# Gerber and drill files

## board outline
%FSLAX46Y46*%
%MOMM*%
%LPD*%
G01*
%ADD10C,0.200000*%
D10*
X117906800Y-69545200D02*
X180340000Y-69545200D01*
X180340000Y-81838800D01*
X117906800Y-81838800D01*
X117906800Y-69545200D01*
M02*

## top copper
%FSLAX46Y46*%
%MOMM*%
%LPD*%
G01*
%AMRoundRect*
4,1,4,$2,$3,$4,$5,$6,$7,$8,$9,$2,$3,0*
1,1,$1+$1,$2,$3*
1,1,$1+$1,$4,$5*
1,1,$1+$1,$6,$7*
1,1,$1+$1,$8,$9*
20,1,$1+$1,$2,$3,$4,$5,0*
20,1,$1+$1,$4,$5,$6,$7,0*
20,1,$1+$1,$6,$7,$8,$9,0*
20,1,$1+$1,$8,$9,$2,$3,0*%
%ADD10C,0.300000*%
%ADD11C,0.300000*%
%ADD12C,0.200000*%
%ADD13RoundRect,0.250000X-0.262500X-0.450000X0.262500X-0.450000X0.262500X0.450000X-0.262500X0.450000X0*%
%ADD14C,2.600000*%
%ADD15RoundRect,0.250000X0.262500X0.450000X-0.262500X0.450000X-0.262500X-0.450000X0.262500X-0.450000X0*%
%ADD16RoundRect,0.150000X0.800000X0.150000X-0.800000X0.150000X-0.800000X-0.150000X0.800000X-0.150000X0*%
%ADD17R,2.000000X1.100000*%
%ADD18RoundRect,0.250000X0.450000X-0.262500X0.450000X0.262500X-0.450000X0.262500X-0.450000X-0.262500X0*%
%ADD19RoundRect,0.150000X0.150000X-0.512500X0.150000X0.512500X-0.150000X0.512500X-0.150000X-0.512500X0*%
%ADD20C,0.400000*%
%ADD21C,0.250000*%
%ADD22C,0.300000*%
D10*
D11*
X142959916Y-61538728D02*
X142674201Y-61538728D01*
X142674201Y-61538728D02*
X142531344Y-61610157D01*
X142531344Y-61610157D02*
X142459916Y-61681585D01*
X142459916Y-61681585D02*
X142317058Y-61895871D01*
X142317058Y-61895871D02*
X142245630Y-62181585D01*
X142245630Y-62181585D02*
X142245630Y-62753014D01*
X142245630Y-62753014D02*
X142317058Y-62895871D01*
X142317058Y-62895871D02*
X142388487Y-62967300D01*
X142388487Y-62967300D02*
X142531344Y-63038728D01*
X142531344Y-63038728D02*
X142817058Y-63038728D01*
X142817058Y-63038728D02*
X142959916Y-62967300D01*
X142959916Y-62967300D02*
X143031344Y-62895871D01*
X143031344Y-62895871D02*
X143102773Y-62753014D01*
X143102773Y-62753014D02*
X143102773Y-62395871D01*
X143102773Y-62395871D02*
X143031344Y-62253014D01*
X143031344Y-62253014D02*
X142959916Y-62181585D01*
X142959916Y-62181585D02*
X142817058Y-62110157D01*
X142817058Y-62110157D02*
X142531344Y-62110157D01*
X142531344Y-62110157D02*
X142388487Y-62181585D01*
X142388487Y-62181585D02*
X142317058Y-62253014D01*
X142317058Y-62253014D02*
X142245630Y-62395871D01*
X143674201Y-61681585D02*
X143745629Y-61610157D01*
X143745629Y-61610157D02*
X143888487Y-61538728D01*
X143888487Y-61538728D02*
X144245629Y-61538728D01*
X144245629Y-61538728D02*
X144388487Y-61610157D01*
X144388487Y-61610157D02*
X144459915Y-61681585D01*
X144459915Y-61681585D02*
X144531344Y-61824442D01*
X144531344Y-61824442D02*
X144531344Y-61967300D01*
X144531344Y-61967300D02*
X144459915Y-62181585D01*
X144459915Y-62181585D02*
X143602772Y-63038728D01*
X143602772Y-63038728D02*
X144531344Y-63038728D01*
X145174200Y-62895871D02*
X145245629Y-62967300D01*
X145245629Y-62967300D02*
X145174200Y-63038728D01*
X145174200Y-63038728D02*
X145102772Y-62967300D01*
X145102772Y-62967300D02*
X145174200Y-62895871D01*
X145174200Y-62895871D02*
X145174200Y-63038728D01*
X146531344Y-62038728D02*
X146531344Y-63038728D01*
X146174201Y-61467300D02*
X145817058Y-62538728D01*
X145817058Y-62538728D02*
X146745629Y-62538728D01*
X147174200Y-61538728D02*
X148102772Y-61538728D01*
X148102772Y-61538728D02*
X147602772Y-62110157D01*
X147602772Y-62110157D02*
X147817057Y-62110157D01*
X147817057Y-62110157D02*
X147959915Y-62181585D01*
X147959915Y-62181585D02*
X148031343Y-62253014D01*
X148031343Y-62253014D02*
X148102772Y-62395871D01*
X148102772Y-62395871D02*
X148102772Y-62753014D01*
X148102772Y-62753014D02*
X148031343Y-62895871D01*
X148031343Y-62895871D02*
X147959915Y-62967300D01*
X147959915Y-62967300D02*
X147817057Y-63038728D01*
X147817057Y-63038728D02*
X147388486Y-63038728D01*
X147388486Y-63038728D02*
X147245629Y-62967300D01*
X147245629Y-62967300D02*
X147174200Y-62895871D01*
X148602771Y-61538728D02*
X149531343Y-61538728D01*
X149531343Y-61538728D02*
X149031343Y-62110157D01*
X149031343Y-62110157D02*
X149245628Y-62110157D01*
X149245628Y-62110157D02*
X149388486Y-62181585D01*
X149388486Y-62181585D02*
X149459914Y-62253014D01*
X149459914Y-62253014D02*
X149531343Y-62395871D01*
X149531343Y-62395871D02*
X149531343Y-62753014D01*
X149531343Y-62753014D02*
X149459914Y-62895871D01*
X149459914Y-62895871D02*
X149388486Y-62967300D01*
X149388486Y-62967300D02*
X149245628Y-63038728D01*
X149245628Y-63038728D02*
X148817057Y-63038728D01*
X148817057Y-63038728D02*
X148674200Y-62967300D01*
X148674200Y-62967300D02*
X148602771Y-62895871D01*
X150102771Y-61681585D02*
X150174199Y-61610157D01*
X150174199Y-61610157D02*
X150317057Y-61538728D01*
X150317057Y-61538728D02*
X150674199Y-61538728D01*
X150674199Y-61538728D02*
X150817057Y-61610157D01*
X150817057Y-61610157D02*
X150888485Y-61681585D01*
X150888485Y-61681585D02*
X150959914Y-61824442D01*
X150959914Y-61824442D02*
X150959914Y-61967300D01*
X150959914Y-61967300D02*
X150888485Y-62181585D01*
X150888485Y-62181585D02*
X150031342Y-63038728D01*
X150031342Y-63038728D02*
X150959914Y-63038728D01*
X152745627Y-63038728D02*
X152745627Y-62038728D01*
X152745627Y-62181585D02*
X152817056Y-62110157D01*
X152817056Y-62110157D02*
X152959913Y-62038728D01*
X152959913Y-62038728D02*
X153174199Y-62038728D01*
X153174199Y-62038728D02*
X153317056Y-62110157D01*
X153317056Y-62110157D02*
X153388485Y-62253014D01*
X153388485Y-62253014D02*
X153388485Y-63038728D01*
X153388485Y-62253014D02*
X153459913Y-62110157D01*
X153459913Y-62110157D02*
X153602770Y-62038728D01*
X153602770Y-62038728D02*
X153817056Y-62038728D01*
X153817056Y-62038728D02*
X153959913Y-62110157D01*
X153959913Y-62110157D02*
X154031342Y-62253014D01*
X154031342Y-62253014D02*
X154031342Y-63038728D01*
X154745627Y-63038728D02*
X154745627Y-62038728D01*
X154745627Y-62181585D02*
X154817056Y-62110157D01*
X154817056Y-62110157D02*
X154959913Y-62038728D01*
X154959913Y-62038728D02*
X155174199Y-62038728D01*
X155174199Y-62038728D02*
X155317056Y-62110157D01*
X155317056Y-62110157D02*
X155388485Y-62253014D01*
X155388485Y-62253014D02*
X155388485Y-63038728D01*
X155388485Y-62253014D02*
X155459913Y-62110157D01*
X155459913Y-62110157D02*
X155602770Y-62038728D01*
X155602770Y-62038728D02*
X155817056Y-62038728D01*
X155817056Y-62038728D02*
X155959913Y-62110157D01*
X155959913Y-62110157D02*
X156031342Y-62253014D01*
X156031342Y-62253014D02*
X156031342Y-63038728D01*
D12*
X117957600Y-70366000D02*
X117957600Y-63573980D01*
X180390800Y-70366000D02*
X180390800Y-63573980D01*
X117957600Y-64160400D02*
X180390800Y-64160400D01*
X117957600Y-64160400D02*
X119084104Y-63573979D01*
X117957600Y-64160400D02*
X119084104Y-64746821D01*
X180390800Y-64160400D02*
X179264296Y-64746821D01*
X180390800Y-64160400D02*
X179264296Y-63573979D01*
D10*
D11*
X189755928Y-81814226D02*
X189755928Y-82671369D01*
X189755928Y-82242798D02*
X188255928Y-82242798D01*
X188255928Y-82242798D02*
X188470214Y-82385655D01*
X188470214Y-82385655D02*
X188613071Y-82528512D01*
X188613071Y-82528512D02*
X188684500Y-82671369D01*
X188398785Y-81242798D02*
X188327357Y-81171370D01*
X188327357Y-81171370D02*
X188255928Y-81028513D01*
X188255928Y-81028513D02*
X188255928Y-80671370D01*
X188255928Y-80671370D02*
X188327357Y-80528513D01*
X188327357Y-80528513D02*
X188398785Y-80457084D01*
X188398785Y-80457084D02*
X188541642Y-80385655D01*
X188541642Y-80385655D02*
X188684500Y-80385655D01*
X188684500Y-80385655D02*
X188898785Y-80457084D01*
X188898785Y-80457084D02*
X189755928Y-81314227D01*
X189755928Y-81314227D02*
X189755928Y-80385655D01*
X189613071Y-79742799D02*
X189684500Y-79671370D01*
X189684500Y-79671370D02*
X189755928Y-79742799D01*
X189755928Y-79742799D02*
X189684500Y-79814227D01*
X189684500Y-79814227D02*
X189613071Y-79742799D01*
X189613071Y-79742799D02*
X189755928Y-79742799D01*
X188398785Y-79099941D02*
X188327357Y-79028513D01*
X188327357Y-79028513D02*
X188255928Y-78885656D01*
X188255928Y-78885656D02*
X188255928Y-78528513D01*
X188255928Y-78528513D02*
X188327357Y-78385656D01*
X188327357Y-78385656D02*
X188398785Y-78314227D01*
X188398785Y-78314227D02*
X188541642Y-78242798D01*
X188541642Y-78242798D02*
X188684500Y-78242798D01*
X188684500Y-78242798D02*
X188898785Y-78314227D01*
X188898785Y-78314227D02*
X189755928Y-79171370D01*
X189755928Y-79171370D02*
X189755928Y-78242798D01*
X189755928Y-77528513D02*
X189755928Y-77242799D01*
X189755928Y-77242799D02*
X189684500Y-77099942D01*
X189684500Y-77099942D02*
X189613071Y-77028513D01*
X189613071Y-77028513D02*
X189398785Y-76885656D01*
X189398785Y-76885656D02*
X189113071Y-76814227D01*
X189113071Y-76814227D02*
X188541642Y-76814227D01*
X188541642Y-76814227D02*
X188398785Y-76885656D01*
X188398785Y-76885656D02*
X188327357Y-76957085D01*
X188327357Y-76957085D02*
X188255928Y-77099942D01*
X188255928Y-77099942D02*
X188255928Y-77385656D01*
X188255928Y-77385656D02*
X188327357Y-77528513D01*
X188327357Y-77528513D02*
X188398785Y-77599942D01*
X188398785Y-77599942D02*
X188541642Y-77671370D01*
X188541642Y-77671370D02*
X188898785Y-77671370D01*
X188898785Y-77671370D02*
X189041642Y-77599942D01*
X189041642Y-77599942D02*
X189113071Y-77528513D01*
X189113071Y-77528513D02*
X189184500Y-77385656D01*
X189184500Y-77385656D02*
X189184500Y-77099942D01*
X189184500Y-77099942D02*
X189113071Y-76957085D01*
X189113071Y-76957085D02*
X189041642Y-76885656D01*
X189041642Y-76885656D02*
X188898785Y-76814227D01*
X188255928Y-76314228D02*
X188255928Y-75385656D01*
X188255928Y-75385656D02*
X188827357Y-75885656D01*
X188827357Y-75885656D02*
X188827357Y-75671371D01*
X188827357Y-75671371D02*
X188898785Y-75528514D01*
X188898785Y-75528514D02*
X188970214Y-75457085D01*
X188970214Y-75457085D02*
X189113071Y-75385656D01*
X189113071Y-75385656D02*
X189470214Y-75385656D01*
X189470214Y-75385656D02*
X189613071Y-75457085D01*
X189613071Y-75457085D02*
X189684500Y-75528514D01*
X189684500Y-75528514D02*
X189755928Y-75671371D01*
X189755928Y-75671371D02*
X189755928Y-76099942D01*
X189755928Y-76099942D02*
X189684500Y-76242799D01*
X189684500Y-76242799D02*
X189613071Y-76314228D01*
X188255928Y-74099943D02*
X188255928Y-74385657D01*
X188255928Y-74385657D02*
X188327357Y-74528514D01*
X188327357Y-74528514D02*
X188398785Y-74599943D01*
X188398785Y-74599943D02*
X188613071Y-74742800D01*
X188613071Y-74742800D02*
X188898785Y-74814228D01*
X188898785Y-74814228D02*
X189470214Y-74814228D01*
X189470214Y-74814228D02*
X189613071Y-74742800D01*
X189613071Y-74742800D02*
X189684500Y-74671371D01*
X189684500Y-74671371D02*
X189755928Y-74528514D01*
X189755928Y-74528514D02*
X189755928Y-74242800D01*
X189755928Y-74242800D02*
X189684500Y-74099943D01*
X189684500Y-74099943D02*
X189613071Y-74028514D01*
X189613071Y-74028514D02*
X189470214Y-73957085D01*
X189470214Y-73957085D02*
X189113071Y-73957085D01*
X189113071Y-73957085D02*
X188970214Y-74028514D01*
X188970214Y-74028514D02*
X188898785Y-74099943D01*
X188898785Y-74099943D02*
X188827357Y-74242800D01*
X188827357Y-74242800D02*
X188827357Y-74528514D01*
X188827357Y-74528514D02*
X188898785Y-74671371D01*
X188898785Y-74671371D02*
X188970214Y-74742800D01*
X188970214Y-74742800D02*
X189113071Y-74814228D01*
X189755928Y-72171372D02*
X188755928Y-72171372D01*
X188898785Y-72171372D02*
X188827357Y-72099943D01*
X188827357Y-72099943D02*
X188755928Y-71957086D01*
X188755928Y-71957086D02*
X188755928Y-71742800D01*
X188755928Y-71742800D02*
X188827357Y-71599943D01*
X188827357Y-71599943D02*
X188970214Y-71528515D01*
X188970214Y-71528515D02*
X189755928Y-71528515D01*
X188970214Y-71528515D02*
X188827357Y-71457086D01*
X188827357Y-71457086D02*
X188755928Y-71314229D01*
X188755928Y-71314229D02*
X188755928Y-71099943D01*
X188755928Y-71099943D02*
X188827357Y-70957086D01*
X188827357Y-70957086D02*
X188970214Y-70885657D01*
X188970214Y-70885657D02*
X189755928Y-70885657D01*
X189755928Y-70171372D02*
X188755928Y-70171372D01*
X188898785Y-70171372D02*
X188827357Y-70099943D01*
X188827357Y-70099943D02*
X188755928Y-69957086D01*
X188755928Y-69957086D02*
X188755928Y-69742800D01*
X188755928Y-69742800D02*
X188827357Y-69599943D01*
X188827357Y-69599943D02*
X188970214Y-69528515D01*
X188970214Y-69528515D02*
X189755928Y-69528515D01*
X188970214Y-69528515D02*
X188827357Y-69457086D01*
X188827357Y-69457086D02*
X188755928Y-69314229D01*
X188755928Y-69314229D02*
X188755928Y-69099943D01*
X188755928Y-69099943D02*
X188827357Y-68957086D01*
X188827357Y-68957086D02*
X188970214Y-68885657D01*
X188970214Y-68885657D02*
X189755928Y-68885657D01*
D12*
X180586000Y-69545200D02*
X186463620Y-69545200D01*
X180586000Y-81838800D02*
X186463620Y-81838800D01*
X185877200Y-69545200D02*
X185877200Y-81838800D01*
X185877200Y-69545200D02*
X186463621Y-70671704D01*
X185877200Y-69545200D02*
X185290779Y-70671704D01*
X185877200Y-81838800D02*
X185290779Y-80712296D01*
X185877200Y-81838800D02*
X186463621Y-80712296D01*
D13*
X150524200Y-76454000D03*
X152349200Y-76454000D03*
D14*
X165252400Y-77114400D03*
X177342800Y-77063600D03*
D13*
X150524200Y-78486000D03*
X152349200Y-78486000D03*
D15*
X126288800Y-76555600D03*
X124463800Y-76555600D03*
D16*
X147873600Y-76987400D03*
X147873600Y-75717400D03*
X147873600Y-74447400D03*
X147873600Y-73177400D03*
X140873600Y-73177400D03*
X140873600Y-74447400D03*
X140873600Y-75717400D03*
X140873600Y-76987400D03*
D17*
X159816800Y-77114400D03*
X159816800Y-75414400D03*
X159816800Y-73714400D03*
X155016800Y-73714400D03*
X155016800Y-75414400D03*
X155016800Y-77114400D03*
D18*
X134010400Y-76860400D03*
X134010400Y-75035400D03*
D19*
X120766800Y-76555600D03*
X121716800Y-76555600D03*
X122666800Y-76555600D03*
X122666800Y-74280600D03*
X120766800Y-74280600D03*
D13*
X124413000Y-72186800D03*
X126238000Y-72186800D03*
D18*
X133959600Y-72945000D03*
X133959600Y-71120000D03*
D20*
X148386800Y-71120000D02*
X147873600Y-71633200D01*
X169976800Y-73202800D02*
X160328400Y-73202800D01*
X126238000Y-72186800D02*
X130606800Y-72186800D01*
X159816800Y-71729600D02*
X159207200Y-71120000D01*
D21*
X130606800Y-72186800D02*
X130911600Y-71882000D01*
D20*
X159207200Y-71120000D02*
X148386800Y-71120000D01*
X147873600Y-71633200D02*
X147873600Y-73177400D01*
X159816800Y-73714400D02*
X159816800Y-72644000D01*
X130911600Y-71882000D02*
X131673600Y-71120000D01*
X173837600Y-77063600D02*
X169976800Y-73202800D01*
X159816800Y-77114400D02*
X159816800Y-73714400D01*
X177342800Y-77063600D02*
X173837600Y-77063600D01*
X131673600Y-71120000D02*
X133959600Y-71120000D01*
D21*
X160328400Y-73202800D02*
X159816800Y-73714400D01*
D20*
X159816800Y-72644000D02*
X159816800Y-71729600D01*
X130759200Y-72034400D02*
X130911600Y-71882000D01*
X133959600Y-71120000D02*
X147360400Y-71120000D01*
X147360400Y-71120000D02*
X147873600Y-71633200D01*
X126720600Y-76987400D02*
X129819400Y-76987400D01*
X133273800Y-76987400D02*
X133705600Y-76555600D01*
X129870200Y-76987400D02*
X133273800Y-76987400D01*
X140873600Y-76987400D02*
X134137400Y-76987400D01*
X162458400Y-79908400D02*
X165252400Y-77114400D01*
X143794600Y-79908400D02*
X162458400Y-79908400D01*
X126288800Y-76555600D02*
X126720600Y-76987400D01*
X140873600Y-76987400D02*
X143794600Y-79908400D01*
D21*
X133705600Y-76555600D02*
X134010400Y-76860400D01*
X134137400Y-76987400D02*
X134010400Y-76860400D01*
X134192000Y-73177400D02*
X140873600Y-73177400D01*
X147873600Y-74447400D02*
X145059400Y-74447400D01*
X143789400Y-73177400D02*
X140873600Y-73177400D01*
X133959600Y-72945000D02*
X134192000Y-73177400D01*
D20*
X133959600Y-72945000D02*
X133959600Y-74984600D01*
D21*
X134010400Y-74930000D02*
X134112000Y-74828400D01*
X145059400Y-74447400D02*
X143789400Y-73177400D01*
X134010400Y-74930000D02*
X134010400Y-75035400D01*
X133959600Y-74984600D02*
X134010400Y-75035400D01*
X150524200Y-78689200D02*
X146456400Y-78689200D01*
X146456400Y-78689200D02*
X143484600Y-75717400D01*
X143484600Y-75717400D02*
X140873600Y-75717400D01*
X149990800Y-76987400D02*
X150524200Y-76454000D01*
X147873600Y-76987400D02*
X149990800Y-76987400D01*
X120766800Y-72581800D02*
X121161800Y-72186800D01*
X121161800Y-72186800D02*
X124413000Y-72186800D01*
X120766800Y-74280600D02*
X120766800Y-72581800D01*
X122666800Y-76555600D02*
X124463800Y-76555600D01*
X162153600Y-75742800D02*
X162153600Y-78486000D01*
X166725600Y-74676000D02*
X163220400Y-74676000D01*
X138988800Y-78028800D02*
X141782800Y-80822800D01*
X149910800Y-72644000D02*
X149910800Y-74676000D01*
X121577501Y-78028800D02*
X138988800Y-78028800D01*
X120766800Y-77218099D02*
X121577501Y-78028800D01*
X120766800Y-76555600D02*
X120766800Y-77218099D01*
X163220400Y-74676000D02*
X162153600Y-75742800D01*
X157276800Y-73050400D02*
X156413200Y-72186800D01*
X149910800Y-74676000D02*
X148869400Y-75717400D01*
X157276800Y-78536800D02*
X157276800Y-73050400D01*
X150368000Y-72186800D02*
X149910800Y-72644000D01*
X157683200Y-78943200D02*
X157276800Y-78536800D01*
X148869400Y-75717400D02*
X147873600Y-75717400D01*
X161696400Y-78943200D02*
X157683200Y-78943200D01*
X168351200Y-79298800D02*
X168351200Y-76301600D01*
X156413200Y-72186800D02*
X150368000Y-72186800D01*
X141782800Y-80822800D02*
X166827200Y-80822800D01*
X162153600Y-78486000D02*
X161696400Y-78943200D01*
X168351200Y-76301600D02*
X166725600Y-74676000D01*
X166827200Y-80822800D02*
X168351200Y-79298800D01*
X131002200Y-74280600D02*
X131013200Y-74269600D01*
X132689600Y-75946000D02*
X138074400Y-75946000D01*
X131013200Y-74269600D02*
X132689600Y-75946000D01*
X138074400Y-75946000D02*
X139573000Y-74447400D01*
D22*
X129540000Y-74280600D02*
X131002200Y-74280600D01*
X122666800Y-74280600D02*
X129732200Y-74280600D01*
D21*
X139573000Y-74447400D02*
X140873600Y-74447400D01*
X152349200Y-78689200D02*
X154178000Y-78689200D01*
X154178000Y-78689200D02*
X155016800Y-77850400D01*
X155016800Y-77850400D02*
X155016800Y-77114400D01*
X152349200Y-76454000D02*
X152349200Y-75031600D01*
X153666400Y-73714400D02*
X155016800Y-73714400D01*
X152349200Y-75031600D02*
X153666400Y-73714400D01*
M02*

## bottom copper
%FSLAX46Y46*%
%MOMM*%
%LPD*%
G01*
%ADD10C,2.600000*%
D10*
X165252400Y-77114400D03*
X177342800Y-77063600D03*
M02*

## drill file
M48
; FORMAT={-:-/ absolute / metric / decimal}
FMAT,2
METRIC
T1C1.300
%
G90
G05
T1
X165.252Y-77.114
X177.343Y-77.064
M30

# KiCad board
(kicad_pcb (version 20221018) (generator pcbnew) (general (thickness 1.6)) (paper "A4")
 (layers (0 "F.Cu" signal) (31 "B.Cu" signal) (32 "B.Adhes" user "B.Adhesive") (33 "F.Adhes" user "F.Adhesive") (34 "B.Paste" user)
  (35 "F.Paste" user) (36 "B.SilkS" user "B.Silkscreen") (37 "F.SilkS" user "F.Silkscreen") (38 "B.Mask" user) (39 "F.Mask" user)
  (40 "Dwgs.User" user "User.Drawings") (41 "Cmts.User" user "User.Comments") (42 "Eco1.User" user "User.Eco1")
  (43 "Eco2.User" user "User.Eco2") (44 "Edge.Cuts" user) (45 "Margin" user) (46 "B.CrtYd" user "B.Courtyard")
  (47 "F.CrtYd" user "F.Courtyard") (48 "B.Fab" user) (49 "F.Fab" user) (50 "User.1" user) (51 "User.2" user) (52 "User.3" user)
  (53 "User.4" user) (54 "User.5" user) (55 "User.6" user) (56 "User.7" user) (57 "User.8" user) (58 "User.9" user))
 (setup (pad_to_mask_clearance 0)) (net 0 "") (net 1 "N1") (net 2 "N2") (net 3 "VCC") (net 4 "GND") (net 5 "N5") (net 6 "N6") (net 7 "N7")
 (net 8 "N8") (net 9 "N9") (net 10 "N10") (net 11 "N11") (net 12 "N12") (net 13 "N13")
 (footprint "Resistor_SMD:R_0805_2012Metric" (layer "F.Cu") (at 151.4367 76.454)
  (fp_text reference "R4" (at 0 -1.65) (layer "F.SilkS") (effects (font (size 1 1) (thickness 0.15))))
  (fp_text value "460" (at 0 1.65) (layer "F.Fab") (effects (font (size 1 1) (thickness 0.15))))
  (pad "1" smd roundrect (at -0.9125 0) (size 1.025 1.4) (layers "F.Cu" "F.Paste" "F.Mask") (roundrect_rratio 0.243902) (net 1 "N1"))
  (pad "2" smd roundrect (at 0.9125 0) (size 1.025 1.4) (layers "F.Cu" "F.Paste" "F.Mask") (roundrect_rratio 0.243902) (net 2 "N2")))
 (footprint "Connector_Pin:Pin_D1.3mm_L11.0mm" (layer "F.Cu") (at 165.2524 77.1144)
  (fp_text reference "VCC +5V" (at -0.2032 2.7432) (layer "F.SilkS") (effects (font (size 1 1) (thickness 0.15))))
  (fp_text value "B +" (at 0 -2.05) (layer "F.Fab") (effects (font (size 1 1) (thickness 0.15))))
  (pad "1" thru_hole circle (at 0 0) (size 2.6 2.6) (drill 1.3) (layers "*.Cu" "*.Mask") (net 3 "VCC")))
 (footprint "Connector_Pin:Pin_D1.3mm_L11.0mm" (layer "F.Cu") (at 177.3428 77.0636)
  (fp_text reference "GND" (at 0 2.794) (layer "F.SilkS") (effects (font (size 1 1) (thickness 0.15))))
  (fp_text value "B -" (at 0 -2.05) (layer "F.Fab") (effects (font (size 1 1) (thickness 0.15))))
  (pad "1" thru_hole circle (at 0 0) (size 2.6 2.6) (drill 1.3) (layers "*.Cu" "*.Mask") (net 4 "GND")))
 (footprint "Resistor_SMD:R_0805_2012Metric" (layer "F.Cu") (at 151.4367 78.486)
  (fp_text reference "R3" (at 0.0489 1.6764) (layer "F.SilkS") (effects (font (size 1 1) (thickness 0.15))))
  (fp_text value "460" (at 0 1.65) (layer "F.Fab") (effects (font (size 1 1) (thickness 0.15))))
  (pad "1" smd roundrect (at -0.9125 0) (size 1.025 1.4) (layers "F.Cu" "F.Paste" "F.Mask") (roundrect_rratio 0.243902) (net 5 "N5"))
  (pad "2" smd roundrect (at 0.9125 0) (size 1.025 1.4) (layers "F.Cu" "F.Paste" "F.Mask") (roundrect_rratio 0.243902) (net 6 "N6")))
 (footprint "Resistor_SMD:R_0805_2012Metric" (layer "F.Cu") (at 125.3763 76.5556 180)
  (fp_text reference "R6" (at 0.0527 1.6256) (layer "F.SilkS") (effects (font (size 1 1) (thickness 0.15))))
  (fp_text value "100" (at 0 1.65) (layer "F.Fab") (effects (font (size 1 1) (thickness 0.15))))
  (pad "1" smd roundrect (at -0.9125 0 180) (size 1.025 1.4) (layers "F.Cu" "F.Paste" "F.Mask") (roundrect_rratio 0.243902) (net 3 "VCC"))
  (pad "2" smd roundrect (at 0.9125 0 180) (size 1.025 1.4) (layers "F.Cu" "F.Paste" "F.Mask") (roundrect_rratio 0.243902) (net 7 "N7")))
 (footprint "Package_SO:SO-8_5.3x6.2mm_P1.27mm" (layer "F.Cu") (at 144.3736 75.0824 180)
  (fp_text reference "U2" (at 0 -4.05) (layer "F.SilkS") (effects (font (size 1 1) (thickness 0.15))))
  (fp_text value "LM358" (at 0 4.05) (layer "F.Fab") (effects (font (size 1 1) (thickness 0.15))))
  (pad "1" smd roundrect (at -3.5 -1.905 180) (size 1.9 0.6) (layers "F.Cu" "F.Paste" "F.Mask") (roundrect_rratio 0.25) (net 1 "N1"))
  (pad "2" smd roundrect (at -3.5 -0.635 180) (size 1.9 0.6) (layers "F.Cu" "F.Paste" "F.Mask") (roundrect_rratio 0.25) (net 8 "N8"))
  (pad "3" smd roundrect (at -3.5 0.635 180) (size 1.9 0.6) (layers "F.Cu" "F.Paste" "F.Mask") (roundrect_rratio 0.25) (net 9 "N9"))
  (pad "4" smd roundrect (at -3.5 1.905 180) (size 1.9 0.6) (layers "F.Cu" "F.Paste" "F.Mask") (roundrect_rratio 0.25) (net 4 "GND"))
  (pad "5" smd roundrect (at 3.5 1.905 180) (size 1.9 0.6) (layers "F.Cu" "F.Paste" "F.Mask") (roundrect_rratio 0.25) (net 9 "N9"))
  (pad "6" smd roundrect (at 3.5 0.635 180) (size 1.9 0.6) (layers "F.Cu" "F.Paste" "F.Mask") (roundrect_rratio 0.25) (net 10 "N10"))
  (pad "7" smd roundrect (at 3.5 -0.635 180) (size 1.9 0.6) (layers "F.Cu" "F.Paste" "F.Mask") (roundrect_rratio 0.25) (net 5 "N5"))
  (pad "8" smd roundrect (at 3.5 -1.905 180) (size 1.9 0.6) (layers "F.Cu" "F.Paste" "F.Mask") (roundrect_rratio 0.25) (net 3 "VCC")))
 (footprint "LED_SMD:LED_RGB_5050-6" (layer "F.Cu") (at 157.4168 75.4144 180)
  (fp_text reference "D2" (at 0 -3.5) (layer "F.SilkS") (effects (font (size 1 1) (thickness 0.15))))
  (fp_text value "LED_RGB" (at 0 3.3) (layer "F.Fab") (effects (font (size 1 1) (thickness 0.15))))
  (pad "1" smd rect (at -2.4 -1.7 270) (size 1.1 2) (layers "F.Cu" "F.Paste" "F.Mask") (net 4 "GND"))
  (pad "2" smd rect (at -2.4 0 270) (size 1.1 2) (layers "F.Cu" "F.Paste" "F.Mask") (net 4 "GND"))
  (pad "3" smd rect (at -2.4 1.7 270) (size 1.1 2) (layers "F.Cu" "F.Paste" "F.Mask") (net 4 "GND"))
  (pad "4" smd rect (at 2.4 1.7 270) (size 1.1 2) (layers "F.Cu" "F.Paste" "F.Mask") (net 2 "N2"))
  (pad "5" smd rect (at 2.4 0 270) (size 1.1 2) (layers "F.Cu" "F.Paste" "F.Mask") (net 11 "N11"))
  (pad "6" smd rect (at 2.4 -1.7 270) (size 1.1 2) (layers "F.Cu" "F.Paste" "F.Mask") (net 6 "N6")))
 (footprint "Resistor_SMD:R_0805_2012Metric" (layer "F.Cu") (at 134.0104 75.9479 90)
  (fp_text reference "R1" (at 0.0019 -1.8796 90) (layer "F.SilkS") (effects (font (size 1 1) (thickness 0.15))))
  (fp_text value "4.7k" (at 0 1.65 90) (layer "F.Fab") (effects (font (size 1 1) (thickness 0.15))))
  (pad "1" smd roundrect (at -0.9125 0 90) (size 1.025 1.4) (layers "F.Cu" "F.Paste" "F.Mask") (roundrect_rratio 0.243902) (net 3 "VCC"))
  (pad "2" smd roundrect (at 0.9125 0 90) (size 1.025 1.4) (layers "F.Cu" "F.Paste" "F.Mask") (roundrect_rratio 0.243902) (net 9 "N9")))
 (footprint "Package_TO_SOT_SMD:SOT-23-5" (layer "F.Cu") (at 121.7168 75.4181 90)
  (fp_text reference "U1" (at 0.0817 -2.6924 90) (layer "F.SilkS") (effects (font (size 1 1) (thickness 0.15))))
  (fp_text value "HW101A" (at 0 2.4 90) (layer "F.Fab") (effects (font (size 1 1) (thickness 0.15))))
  (pad "1" smd roundrect (at -1.1375 -0.95 90) (size 1.325 0.6) (layers "F.Cu" "F.Paste" "F.Mask") (roundrect_rratio 0.25) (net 8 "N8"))
  (pad "2" smd roundrect (at -1.1375 0 90) (size 1.325 0.6) (layers "F.Cu" "F.Paste" "F.Mask") (roundrect_rratio 0.25) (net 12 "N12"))
  (pad "3" smd roundrect (at -1.1375 0.95 90) (size 1.325 0.6) (layers "F.Cu" "F.Paste" "F.Mask") (roundrect_rratio 0.25) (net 7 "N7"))
  (pad "4" smd roundrect (at 1.1375 0.95 90) (size 1.325 0.6) (layers "F.Cu" "F.Paste" "F.Mask") (roundrect_rratio 0.25) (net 10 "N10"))
  (pad "5" smd roundrect (at 1.1375 -0.95 90) (size 1.325 0.6) (layers "F.Cu" "F.Paste" "F.Mask") (roundrect_rratio 0.25) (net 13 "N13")))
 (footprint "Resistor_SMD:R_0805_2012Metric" (layer "F.Cu") (at 125.3255 72.1868)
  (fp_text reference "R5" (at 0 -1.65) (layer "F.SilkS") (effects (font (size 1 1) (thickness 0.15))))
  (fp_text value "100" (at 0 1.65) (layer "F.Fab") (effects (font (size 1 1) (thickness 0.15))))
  (pad "1" smd roundrect (at -0.9125 0) (size 1.025 1.4) (layers "F.Cu" "F.Paste" "F.Mask") (roundrect_rratio 0.243902) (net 13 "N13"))
  (pad "2" smd roundrect (at 0.9125 0) (size 1.025 1.4) (layers "F.Cu" "F.Paste" "F.Mask") (roundrect_rratio 0.243902) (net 4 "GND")))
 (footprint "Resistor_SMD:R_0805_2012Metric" (layer "F.Cu") (at 133.9596 72.0325 90)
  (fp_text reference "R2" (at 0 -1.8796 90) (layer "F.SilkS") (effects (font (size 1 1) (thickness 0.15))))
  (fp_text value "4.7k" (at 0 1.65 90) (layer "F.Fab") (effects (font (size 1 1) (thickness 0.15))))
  (pad "1" smd roundrect (at -0.9125 0 90) (size 1.025 1.4) (layers "F.Cu" "F.Paste" "F.Mask") (roundrect_rratio 0.243902) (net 9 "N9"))
  (pad "2" smd roundrect (at 0.9125 0 90) (size 1.025 1.4) (layers "F.Cu" "F.Paste" "F.Mask") (roundrect_rratio 0.243902) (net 4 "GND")))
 (gr_rect (start 117.9068 69.5452) (end 180.34 81.8388) (stroke (width 0.2) (type default)) (fill none) (layer "Edge.Cuts"))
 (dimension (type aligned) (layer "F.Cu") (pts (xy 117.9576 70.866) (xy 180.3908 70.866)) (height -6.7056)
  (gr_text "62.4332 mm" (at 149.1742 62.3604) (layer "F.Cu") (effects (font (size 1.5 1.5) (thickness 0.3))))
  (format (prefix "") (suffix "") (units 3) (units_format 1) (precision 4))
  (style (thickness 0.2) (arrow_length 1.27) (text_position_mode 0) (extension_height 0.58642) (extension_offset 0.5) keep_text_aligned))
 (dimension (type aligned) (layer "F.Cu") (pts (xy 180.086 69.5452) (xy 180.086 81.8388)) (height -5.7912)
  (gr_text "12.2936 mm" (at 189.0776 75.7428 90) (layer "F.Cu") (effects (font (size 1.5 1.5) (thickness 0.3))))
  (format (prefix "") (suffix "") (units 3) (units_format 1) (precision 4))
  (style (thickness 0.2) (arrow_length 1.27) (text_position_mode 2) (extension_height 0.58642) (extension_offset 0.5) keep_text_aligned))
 (segment (start 148.3868 71.12) (end 147.8736 71.6332) (width 0.4) (layer "F.Cu") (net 4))
 (segment (start 169.9768 73.2028) (end 160.3284 73.2028) (width 0.4) (layer "F.Cu") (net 4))
 (segment (start 126.238 72.1868) (end 130.6068 72.1868) (width 0.4) (layer "F.Cu") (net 4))
 (segment (start 159.8168 71.7296) (end 159.2072 71.12) (width 0.4) (layer "F.Cu") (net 4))
 (segment (start 130.6068 72.1868) (end 130.9116 71.882) (width 0.25) (layer "F.Cu") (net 4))
 (segment (start 159.2072 71.12) (end 148.3868 71.12) (width 0.4) (layer "F.Cu") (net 4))
 (segment (start 147.8736 71.6332) (end 147.8736 73.1774) (width 0.4) (layer "F.Cu") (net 4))
 (segment (start 159.8168 73.7144) (end 159.8168 72.644) (width 0.4) (layer "F.Cu") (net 4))
 (segment (start 130.9116 71.882) (end 131.6736 71.12) (width 0.4) (layer "F.Cu") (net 4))
 (segment (start 173.8376 77.0636) (end 169.9768 73.2028) (width 0.4) (layer "F.Cu") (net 4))
 (segment (start 159.8168 77.1144) (end 159.8168 73.7144) (width 0.4) (layer "F.Cu") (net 4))
 (segment (start 177.3428 77.0636) (end 173.8376 77.0636) (width 0.4) (layer "F.Cu") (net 4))
 (segment (start 131.6736 71.12) (end 133.9596 71.12) (width 0.4) (layer "F.Cu") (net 4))
 (segment (start 160.3284 73.2028) (end 159.8168 73.7144) (width 0.25) (layer "F.Cu") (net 4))
 (segment (start 159.8168 72.644) (end 159.8168 71.7296) (width 0.4) (layer "F.Cu") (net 4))
 (segment (start 130.7592 72.0344) (end 130.9116 71.882) (width 0.4) (layer "F.Cu") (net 4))
 (segment (start 133.9596 71.12) (end 147.3604 71.12) (width 0.4) (layer "F.Cu") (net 4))
 (segment (start 147.3604 71.12) (end 147.8736 71.6332) (width 0.4) (layer "F.Cu") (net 4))
 (segment (start 126.7206 76.9874) (end 129.8194 76.9874) (width 0.4) (layer "F.Cu") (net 3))
 (segment (start 133.2738 76.9874) (end 133.7056 76.5556) (width 0.4) (layer "F.Cu") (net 3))
 (segment (start 129.8702 76.9874) (end 133.2738 76.9874) (width 0.4) (layer "F.Cu") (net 3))
 (segment (start 140.8736 76.9874) (end 134.1374 76.9874) (width 0.4) (layer "F.Cu") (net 3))
 (segment (start 162.4584 79.9084) (end 165.2524 77.1144) (width 0.4) (layer "F.Cu") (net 3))
 (segment (start 143.7946 79.9084) (end 162.4584 79.9084) (width 0.4) (layer "F.Cu") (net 3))
 (segment (start 126.2888 76.5556) (end 126.7206 76.9874) (width 0.4) (layer "F.Cu") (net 3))
 (segment (start 140.8736 76.9874) (end 143.7946 79.9084) (width 0.4) (layer "F.Cu") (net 3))
 (segment (start 133.7056 76.5556) (end 134.0104 76.8604) (width 0.25) (layer "F.Cu") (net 3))
 (segment (start 134.1374 76.9874) (end 134.0104 76.8604) (width 0.25) (layer "F.Cu") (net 3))
 (segment (start 134.192 73.1774) (end 140.8736 73.1774) (width 0.25) (layer "F.Cu") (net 9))
 (segment (start 147.8736 74.4474) (end 145.0594 74.4474) (width 0.25) (layer "F.Cu") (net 9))
 (segment (start 143.7894 73.1774) (end 140.8736 73.1774) (width 0.25) (layer "F.Cu") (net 9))
 (segment (start 133.9596 72.945) (end 134.192 73.1774) (width 0.25) (layer "F.Cu") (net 9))
 (segment (start 133.9596 72.945) (end 133.9596 74.9846) (width 0.4) (layer "F.Cu") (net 9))
 (segment (start 134.0104 74.93) (end 134.112 74.8284) (width 0.25) (layer "F.Cu") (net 9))
 (segment (start 145.0594 74.4474) (end 143.7894 73.1774) (width 0.25) (layer "F.Cu") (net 9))
 (segment (start 134.0104 74.93) (end 134.0104 75.0354) (width 0.25) (layer "F.Cu") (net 9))
 (segment (start 133.9596 74.9846) (end 134.0104 75.0354) (width 0.25) (layer "F.Cu") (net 9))
 (segment (start 150.5242 78.6892) (end 146.4564 78.6892) (width 0.25) (layer "F.Cu") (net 5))
 (segment (start 146.4564 78.6892) (end 143.4846 75.7174) (width 0.25) (layer "F.Cu") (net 5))
 (segment (start 143.4846 75.7174) (end 140.8736 75.7174) (width 0.25) (layer "F.Cu") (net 5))
 (segment (start 149.9908 76.9874) (end 150.5242 76.454) (width 0.25) (layer "F.Cu") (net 1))
 (segment (start 147.8736 76.9874) (end 149.9908 76.9874) (width 0.25) (layer "F.Cu") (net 1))
 (segment (start 120.7668 72.5818) (end 121.1618 72.1868) (width 0.25) (layer "F.Cu") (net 13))
 (segment (start 121.1618 72.1868) (end 124.413 72.1868) (width 0.25) (layer "F.Cu") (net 13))
 (segment (start 120.7668 74.2806) (end 120.7668 72.5818) (width 0.25) (layer "F.Cu") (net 13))
 (segment (start 122.6668 76.5556) (end 124.4638 76.5556) (width 0.25) (layer "F.Cu") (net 7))
 (segment (start 162.1536 75.7428) (end 162.1536 78.486) (width 0.25) (layer "F.Cu") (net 8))
 (segment (start 166.7256 74.676) (end 163.2204 74.676) (width 0.25) (layer "F.Cu") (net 8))
 (segment (start 138.9888 78.0288) (end 141.7828 80.8228) (width 0.25) (layer "F.Cu") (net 8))
 (segment (start 149.9108 72.644) (end 149.9108 74.676) (width 0.25) (layer "F.Cu") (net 8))
 (segment (start 121.577501 78.0288) (end 138.9888 78.0288) (width 0.25) (layer "F.Cu") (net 8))
 (segment (start 120.7668 77.218099) (end 121.577501 78.0288) (width 0.25) (layer "F.Cu") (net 8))
 (segment (start 120.7668 76.5556) (end 120.7668 77.218099) (width 0.25) (layer "F.Cu") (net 8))
 (segment (start 163.2204 74.676) (end 162.1536 75.7428) (width 0.25) (layer "F.Cu") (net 8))
 (segment (start 157.2768 73.0504) (end 156.4132 72.1868) (width 0.25) (layer "F.Cu") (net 8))
 (segment (start 149.9108 74.676) (end 148.8694 75.7174) (width 0.25) (layer "F.Cu") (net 8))
 (segment (start 157.2768 78.5368) (end 157.2768 73.0504) (width 0.25) (layer "F.Cu") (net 8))
 (segment (start 150.368 72.1868) (end 149.9108 72.644) (width 0.25) (layer "F.Cu") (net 8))
 (segment (start 157.6832 78.9432) (end 157.2768 78.5368) (width 0.25) (layer "F.Cu") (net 8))
 (segment (start 148.8694 75.7174) (end 147.8736 75.7174) (width 0.25) (layer "F.Cu") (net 8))
 (segment (start 161.6964 78.9432) (end 157.6832 78.9432) (width 0.25) (layer "F.Cu") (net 8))
 (segment (start 168.3512 79.2988) (end 168.3512 76.3016) (width 0.25) (layer "F.Cu") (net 8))
 (segment (start 156.4132 72.1868) (end 150.368 72.1868) (width 0.25) (layer "F.Cu") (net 8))
 (segment (start 141.7828 80.8228) (end 166.8272 80.8228) (width 0.25) (layer "F.Cu") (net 8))
 (segment (start 162.1536 78.486) (end 161.6964 78.9432) (width 0.25) (layer "F.Cu") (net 8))
 (segment (start 168.3512 76.3016) (end 166.7256 74.676) (width 0.25) (layer "F.Cu") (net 8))
 (segment (start 166.8272 80.8228) (end 168.3512 79.2988) (width 0.25) (layer "F.Cu") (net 8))
 (segment (start 131.0022 74.2806) (end 131.0132 74.2696) (width 0.25) (layer "F.Cu") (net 10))
 (segment (start 132.6896 75.946) (end 138.0744 75.946) (width 0.25) (layer "F.Cu") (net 10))
 (segment (start 131.0132 74.2696) (end 132.6896 75.946) (width 0.25) (layer "F.Cu") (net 10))
 (segment (start 138.0744 75.946) (end 139.573 74.4474) (width 0.25) (layer "F.Cu") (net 10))
 (segment (start 129.54 74.2806) (end 131.0022 74.2806) (width 0.3) (layer "F.Cu") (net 10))
 (segment (start 122.6668 74.2806) (end 129.7322 74.2806) (width 0.3) (layer "F.Cu") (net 10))
 (segment (start 139.573 74.4474) (end 140.8736 74.4474) (width 0.25) (layer "F.Cu") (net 10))
 (segment (start 152.3492 78.6892) (end 154.178 78.6892) (width 0.25) (layer "F.Cu") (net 6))
 (segment (start 154.178 78.6892) (end 155.0168 77.8504) (width 0.25) (layer "F.Cu") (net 6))
 (segment (start 155.0168 77.8504) (end 155.0168 77.1144) (width 0.25) (layer "F.Cu") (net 6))
 (segment (start 152.3492 76.454) (end 152.3492 75.0316) (width 0.25) (layer "F.Cu") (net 2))
 (segment (start 153.6664 73.7144) (end 155.0168 73.7144) (width 0.25) (layer "F.Cu") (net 2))
 (segment (start 152.3492 75.0316) (end 153.6664 73.7144) (width 0.25) (layer "F.Cu") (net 2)))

